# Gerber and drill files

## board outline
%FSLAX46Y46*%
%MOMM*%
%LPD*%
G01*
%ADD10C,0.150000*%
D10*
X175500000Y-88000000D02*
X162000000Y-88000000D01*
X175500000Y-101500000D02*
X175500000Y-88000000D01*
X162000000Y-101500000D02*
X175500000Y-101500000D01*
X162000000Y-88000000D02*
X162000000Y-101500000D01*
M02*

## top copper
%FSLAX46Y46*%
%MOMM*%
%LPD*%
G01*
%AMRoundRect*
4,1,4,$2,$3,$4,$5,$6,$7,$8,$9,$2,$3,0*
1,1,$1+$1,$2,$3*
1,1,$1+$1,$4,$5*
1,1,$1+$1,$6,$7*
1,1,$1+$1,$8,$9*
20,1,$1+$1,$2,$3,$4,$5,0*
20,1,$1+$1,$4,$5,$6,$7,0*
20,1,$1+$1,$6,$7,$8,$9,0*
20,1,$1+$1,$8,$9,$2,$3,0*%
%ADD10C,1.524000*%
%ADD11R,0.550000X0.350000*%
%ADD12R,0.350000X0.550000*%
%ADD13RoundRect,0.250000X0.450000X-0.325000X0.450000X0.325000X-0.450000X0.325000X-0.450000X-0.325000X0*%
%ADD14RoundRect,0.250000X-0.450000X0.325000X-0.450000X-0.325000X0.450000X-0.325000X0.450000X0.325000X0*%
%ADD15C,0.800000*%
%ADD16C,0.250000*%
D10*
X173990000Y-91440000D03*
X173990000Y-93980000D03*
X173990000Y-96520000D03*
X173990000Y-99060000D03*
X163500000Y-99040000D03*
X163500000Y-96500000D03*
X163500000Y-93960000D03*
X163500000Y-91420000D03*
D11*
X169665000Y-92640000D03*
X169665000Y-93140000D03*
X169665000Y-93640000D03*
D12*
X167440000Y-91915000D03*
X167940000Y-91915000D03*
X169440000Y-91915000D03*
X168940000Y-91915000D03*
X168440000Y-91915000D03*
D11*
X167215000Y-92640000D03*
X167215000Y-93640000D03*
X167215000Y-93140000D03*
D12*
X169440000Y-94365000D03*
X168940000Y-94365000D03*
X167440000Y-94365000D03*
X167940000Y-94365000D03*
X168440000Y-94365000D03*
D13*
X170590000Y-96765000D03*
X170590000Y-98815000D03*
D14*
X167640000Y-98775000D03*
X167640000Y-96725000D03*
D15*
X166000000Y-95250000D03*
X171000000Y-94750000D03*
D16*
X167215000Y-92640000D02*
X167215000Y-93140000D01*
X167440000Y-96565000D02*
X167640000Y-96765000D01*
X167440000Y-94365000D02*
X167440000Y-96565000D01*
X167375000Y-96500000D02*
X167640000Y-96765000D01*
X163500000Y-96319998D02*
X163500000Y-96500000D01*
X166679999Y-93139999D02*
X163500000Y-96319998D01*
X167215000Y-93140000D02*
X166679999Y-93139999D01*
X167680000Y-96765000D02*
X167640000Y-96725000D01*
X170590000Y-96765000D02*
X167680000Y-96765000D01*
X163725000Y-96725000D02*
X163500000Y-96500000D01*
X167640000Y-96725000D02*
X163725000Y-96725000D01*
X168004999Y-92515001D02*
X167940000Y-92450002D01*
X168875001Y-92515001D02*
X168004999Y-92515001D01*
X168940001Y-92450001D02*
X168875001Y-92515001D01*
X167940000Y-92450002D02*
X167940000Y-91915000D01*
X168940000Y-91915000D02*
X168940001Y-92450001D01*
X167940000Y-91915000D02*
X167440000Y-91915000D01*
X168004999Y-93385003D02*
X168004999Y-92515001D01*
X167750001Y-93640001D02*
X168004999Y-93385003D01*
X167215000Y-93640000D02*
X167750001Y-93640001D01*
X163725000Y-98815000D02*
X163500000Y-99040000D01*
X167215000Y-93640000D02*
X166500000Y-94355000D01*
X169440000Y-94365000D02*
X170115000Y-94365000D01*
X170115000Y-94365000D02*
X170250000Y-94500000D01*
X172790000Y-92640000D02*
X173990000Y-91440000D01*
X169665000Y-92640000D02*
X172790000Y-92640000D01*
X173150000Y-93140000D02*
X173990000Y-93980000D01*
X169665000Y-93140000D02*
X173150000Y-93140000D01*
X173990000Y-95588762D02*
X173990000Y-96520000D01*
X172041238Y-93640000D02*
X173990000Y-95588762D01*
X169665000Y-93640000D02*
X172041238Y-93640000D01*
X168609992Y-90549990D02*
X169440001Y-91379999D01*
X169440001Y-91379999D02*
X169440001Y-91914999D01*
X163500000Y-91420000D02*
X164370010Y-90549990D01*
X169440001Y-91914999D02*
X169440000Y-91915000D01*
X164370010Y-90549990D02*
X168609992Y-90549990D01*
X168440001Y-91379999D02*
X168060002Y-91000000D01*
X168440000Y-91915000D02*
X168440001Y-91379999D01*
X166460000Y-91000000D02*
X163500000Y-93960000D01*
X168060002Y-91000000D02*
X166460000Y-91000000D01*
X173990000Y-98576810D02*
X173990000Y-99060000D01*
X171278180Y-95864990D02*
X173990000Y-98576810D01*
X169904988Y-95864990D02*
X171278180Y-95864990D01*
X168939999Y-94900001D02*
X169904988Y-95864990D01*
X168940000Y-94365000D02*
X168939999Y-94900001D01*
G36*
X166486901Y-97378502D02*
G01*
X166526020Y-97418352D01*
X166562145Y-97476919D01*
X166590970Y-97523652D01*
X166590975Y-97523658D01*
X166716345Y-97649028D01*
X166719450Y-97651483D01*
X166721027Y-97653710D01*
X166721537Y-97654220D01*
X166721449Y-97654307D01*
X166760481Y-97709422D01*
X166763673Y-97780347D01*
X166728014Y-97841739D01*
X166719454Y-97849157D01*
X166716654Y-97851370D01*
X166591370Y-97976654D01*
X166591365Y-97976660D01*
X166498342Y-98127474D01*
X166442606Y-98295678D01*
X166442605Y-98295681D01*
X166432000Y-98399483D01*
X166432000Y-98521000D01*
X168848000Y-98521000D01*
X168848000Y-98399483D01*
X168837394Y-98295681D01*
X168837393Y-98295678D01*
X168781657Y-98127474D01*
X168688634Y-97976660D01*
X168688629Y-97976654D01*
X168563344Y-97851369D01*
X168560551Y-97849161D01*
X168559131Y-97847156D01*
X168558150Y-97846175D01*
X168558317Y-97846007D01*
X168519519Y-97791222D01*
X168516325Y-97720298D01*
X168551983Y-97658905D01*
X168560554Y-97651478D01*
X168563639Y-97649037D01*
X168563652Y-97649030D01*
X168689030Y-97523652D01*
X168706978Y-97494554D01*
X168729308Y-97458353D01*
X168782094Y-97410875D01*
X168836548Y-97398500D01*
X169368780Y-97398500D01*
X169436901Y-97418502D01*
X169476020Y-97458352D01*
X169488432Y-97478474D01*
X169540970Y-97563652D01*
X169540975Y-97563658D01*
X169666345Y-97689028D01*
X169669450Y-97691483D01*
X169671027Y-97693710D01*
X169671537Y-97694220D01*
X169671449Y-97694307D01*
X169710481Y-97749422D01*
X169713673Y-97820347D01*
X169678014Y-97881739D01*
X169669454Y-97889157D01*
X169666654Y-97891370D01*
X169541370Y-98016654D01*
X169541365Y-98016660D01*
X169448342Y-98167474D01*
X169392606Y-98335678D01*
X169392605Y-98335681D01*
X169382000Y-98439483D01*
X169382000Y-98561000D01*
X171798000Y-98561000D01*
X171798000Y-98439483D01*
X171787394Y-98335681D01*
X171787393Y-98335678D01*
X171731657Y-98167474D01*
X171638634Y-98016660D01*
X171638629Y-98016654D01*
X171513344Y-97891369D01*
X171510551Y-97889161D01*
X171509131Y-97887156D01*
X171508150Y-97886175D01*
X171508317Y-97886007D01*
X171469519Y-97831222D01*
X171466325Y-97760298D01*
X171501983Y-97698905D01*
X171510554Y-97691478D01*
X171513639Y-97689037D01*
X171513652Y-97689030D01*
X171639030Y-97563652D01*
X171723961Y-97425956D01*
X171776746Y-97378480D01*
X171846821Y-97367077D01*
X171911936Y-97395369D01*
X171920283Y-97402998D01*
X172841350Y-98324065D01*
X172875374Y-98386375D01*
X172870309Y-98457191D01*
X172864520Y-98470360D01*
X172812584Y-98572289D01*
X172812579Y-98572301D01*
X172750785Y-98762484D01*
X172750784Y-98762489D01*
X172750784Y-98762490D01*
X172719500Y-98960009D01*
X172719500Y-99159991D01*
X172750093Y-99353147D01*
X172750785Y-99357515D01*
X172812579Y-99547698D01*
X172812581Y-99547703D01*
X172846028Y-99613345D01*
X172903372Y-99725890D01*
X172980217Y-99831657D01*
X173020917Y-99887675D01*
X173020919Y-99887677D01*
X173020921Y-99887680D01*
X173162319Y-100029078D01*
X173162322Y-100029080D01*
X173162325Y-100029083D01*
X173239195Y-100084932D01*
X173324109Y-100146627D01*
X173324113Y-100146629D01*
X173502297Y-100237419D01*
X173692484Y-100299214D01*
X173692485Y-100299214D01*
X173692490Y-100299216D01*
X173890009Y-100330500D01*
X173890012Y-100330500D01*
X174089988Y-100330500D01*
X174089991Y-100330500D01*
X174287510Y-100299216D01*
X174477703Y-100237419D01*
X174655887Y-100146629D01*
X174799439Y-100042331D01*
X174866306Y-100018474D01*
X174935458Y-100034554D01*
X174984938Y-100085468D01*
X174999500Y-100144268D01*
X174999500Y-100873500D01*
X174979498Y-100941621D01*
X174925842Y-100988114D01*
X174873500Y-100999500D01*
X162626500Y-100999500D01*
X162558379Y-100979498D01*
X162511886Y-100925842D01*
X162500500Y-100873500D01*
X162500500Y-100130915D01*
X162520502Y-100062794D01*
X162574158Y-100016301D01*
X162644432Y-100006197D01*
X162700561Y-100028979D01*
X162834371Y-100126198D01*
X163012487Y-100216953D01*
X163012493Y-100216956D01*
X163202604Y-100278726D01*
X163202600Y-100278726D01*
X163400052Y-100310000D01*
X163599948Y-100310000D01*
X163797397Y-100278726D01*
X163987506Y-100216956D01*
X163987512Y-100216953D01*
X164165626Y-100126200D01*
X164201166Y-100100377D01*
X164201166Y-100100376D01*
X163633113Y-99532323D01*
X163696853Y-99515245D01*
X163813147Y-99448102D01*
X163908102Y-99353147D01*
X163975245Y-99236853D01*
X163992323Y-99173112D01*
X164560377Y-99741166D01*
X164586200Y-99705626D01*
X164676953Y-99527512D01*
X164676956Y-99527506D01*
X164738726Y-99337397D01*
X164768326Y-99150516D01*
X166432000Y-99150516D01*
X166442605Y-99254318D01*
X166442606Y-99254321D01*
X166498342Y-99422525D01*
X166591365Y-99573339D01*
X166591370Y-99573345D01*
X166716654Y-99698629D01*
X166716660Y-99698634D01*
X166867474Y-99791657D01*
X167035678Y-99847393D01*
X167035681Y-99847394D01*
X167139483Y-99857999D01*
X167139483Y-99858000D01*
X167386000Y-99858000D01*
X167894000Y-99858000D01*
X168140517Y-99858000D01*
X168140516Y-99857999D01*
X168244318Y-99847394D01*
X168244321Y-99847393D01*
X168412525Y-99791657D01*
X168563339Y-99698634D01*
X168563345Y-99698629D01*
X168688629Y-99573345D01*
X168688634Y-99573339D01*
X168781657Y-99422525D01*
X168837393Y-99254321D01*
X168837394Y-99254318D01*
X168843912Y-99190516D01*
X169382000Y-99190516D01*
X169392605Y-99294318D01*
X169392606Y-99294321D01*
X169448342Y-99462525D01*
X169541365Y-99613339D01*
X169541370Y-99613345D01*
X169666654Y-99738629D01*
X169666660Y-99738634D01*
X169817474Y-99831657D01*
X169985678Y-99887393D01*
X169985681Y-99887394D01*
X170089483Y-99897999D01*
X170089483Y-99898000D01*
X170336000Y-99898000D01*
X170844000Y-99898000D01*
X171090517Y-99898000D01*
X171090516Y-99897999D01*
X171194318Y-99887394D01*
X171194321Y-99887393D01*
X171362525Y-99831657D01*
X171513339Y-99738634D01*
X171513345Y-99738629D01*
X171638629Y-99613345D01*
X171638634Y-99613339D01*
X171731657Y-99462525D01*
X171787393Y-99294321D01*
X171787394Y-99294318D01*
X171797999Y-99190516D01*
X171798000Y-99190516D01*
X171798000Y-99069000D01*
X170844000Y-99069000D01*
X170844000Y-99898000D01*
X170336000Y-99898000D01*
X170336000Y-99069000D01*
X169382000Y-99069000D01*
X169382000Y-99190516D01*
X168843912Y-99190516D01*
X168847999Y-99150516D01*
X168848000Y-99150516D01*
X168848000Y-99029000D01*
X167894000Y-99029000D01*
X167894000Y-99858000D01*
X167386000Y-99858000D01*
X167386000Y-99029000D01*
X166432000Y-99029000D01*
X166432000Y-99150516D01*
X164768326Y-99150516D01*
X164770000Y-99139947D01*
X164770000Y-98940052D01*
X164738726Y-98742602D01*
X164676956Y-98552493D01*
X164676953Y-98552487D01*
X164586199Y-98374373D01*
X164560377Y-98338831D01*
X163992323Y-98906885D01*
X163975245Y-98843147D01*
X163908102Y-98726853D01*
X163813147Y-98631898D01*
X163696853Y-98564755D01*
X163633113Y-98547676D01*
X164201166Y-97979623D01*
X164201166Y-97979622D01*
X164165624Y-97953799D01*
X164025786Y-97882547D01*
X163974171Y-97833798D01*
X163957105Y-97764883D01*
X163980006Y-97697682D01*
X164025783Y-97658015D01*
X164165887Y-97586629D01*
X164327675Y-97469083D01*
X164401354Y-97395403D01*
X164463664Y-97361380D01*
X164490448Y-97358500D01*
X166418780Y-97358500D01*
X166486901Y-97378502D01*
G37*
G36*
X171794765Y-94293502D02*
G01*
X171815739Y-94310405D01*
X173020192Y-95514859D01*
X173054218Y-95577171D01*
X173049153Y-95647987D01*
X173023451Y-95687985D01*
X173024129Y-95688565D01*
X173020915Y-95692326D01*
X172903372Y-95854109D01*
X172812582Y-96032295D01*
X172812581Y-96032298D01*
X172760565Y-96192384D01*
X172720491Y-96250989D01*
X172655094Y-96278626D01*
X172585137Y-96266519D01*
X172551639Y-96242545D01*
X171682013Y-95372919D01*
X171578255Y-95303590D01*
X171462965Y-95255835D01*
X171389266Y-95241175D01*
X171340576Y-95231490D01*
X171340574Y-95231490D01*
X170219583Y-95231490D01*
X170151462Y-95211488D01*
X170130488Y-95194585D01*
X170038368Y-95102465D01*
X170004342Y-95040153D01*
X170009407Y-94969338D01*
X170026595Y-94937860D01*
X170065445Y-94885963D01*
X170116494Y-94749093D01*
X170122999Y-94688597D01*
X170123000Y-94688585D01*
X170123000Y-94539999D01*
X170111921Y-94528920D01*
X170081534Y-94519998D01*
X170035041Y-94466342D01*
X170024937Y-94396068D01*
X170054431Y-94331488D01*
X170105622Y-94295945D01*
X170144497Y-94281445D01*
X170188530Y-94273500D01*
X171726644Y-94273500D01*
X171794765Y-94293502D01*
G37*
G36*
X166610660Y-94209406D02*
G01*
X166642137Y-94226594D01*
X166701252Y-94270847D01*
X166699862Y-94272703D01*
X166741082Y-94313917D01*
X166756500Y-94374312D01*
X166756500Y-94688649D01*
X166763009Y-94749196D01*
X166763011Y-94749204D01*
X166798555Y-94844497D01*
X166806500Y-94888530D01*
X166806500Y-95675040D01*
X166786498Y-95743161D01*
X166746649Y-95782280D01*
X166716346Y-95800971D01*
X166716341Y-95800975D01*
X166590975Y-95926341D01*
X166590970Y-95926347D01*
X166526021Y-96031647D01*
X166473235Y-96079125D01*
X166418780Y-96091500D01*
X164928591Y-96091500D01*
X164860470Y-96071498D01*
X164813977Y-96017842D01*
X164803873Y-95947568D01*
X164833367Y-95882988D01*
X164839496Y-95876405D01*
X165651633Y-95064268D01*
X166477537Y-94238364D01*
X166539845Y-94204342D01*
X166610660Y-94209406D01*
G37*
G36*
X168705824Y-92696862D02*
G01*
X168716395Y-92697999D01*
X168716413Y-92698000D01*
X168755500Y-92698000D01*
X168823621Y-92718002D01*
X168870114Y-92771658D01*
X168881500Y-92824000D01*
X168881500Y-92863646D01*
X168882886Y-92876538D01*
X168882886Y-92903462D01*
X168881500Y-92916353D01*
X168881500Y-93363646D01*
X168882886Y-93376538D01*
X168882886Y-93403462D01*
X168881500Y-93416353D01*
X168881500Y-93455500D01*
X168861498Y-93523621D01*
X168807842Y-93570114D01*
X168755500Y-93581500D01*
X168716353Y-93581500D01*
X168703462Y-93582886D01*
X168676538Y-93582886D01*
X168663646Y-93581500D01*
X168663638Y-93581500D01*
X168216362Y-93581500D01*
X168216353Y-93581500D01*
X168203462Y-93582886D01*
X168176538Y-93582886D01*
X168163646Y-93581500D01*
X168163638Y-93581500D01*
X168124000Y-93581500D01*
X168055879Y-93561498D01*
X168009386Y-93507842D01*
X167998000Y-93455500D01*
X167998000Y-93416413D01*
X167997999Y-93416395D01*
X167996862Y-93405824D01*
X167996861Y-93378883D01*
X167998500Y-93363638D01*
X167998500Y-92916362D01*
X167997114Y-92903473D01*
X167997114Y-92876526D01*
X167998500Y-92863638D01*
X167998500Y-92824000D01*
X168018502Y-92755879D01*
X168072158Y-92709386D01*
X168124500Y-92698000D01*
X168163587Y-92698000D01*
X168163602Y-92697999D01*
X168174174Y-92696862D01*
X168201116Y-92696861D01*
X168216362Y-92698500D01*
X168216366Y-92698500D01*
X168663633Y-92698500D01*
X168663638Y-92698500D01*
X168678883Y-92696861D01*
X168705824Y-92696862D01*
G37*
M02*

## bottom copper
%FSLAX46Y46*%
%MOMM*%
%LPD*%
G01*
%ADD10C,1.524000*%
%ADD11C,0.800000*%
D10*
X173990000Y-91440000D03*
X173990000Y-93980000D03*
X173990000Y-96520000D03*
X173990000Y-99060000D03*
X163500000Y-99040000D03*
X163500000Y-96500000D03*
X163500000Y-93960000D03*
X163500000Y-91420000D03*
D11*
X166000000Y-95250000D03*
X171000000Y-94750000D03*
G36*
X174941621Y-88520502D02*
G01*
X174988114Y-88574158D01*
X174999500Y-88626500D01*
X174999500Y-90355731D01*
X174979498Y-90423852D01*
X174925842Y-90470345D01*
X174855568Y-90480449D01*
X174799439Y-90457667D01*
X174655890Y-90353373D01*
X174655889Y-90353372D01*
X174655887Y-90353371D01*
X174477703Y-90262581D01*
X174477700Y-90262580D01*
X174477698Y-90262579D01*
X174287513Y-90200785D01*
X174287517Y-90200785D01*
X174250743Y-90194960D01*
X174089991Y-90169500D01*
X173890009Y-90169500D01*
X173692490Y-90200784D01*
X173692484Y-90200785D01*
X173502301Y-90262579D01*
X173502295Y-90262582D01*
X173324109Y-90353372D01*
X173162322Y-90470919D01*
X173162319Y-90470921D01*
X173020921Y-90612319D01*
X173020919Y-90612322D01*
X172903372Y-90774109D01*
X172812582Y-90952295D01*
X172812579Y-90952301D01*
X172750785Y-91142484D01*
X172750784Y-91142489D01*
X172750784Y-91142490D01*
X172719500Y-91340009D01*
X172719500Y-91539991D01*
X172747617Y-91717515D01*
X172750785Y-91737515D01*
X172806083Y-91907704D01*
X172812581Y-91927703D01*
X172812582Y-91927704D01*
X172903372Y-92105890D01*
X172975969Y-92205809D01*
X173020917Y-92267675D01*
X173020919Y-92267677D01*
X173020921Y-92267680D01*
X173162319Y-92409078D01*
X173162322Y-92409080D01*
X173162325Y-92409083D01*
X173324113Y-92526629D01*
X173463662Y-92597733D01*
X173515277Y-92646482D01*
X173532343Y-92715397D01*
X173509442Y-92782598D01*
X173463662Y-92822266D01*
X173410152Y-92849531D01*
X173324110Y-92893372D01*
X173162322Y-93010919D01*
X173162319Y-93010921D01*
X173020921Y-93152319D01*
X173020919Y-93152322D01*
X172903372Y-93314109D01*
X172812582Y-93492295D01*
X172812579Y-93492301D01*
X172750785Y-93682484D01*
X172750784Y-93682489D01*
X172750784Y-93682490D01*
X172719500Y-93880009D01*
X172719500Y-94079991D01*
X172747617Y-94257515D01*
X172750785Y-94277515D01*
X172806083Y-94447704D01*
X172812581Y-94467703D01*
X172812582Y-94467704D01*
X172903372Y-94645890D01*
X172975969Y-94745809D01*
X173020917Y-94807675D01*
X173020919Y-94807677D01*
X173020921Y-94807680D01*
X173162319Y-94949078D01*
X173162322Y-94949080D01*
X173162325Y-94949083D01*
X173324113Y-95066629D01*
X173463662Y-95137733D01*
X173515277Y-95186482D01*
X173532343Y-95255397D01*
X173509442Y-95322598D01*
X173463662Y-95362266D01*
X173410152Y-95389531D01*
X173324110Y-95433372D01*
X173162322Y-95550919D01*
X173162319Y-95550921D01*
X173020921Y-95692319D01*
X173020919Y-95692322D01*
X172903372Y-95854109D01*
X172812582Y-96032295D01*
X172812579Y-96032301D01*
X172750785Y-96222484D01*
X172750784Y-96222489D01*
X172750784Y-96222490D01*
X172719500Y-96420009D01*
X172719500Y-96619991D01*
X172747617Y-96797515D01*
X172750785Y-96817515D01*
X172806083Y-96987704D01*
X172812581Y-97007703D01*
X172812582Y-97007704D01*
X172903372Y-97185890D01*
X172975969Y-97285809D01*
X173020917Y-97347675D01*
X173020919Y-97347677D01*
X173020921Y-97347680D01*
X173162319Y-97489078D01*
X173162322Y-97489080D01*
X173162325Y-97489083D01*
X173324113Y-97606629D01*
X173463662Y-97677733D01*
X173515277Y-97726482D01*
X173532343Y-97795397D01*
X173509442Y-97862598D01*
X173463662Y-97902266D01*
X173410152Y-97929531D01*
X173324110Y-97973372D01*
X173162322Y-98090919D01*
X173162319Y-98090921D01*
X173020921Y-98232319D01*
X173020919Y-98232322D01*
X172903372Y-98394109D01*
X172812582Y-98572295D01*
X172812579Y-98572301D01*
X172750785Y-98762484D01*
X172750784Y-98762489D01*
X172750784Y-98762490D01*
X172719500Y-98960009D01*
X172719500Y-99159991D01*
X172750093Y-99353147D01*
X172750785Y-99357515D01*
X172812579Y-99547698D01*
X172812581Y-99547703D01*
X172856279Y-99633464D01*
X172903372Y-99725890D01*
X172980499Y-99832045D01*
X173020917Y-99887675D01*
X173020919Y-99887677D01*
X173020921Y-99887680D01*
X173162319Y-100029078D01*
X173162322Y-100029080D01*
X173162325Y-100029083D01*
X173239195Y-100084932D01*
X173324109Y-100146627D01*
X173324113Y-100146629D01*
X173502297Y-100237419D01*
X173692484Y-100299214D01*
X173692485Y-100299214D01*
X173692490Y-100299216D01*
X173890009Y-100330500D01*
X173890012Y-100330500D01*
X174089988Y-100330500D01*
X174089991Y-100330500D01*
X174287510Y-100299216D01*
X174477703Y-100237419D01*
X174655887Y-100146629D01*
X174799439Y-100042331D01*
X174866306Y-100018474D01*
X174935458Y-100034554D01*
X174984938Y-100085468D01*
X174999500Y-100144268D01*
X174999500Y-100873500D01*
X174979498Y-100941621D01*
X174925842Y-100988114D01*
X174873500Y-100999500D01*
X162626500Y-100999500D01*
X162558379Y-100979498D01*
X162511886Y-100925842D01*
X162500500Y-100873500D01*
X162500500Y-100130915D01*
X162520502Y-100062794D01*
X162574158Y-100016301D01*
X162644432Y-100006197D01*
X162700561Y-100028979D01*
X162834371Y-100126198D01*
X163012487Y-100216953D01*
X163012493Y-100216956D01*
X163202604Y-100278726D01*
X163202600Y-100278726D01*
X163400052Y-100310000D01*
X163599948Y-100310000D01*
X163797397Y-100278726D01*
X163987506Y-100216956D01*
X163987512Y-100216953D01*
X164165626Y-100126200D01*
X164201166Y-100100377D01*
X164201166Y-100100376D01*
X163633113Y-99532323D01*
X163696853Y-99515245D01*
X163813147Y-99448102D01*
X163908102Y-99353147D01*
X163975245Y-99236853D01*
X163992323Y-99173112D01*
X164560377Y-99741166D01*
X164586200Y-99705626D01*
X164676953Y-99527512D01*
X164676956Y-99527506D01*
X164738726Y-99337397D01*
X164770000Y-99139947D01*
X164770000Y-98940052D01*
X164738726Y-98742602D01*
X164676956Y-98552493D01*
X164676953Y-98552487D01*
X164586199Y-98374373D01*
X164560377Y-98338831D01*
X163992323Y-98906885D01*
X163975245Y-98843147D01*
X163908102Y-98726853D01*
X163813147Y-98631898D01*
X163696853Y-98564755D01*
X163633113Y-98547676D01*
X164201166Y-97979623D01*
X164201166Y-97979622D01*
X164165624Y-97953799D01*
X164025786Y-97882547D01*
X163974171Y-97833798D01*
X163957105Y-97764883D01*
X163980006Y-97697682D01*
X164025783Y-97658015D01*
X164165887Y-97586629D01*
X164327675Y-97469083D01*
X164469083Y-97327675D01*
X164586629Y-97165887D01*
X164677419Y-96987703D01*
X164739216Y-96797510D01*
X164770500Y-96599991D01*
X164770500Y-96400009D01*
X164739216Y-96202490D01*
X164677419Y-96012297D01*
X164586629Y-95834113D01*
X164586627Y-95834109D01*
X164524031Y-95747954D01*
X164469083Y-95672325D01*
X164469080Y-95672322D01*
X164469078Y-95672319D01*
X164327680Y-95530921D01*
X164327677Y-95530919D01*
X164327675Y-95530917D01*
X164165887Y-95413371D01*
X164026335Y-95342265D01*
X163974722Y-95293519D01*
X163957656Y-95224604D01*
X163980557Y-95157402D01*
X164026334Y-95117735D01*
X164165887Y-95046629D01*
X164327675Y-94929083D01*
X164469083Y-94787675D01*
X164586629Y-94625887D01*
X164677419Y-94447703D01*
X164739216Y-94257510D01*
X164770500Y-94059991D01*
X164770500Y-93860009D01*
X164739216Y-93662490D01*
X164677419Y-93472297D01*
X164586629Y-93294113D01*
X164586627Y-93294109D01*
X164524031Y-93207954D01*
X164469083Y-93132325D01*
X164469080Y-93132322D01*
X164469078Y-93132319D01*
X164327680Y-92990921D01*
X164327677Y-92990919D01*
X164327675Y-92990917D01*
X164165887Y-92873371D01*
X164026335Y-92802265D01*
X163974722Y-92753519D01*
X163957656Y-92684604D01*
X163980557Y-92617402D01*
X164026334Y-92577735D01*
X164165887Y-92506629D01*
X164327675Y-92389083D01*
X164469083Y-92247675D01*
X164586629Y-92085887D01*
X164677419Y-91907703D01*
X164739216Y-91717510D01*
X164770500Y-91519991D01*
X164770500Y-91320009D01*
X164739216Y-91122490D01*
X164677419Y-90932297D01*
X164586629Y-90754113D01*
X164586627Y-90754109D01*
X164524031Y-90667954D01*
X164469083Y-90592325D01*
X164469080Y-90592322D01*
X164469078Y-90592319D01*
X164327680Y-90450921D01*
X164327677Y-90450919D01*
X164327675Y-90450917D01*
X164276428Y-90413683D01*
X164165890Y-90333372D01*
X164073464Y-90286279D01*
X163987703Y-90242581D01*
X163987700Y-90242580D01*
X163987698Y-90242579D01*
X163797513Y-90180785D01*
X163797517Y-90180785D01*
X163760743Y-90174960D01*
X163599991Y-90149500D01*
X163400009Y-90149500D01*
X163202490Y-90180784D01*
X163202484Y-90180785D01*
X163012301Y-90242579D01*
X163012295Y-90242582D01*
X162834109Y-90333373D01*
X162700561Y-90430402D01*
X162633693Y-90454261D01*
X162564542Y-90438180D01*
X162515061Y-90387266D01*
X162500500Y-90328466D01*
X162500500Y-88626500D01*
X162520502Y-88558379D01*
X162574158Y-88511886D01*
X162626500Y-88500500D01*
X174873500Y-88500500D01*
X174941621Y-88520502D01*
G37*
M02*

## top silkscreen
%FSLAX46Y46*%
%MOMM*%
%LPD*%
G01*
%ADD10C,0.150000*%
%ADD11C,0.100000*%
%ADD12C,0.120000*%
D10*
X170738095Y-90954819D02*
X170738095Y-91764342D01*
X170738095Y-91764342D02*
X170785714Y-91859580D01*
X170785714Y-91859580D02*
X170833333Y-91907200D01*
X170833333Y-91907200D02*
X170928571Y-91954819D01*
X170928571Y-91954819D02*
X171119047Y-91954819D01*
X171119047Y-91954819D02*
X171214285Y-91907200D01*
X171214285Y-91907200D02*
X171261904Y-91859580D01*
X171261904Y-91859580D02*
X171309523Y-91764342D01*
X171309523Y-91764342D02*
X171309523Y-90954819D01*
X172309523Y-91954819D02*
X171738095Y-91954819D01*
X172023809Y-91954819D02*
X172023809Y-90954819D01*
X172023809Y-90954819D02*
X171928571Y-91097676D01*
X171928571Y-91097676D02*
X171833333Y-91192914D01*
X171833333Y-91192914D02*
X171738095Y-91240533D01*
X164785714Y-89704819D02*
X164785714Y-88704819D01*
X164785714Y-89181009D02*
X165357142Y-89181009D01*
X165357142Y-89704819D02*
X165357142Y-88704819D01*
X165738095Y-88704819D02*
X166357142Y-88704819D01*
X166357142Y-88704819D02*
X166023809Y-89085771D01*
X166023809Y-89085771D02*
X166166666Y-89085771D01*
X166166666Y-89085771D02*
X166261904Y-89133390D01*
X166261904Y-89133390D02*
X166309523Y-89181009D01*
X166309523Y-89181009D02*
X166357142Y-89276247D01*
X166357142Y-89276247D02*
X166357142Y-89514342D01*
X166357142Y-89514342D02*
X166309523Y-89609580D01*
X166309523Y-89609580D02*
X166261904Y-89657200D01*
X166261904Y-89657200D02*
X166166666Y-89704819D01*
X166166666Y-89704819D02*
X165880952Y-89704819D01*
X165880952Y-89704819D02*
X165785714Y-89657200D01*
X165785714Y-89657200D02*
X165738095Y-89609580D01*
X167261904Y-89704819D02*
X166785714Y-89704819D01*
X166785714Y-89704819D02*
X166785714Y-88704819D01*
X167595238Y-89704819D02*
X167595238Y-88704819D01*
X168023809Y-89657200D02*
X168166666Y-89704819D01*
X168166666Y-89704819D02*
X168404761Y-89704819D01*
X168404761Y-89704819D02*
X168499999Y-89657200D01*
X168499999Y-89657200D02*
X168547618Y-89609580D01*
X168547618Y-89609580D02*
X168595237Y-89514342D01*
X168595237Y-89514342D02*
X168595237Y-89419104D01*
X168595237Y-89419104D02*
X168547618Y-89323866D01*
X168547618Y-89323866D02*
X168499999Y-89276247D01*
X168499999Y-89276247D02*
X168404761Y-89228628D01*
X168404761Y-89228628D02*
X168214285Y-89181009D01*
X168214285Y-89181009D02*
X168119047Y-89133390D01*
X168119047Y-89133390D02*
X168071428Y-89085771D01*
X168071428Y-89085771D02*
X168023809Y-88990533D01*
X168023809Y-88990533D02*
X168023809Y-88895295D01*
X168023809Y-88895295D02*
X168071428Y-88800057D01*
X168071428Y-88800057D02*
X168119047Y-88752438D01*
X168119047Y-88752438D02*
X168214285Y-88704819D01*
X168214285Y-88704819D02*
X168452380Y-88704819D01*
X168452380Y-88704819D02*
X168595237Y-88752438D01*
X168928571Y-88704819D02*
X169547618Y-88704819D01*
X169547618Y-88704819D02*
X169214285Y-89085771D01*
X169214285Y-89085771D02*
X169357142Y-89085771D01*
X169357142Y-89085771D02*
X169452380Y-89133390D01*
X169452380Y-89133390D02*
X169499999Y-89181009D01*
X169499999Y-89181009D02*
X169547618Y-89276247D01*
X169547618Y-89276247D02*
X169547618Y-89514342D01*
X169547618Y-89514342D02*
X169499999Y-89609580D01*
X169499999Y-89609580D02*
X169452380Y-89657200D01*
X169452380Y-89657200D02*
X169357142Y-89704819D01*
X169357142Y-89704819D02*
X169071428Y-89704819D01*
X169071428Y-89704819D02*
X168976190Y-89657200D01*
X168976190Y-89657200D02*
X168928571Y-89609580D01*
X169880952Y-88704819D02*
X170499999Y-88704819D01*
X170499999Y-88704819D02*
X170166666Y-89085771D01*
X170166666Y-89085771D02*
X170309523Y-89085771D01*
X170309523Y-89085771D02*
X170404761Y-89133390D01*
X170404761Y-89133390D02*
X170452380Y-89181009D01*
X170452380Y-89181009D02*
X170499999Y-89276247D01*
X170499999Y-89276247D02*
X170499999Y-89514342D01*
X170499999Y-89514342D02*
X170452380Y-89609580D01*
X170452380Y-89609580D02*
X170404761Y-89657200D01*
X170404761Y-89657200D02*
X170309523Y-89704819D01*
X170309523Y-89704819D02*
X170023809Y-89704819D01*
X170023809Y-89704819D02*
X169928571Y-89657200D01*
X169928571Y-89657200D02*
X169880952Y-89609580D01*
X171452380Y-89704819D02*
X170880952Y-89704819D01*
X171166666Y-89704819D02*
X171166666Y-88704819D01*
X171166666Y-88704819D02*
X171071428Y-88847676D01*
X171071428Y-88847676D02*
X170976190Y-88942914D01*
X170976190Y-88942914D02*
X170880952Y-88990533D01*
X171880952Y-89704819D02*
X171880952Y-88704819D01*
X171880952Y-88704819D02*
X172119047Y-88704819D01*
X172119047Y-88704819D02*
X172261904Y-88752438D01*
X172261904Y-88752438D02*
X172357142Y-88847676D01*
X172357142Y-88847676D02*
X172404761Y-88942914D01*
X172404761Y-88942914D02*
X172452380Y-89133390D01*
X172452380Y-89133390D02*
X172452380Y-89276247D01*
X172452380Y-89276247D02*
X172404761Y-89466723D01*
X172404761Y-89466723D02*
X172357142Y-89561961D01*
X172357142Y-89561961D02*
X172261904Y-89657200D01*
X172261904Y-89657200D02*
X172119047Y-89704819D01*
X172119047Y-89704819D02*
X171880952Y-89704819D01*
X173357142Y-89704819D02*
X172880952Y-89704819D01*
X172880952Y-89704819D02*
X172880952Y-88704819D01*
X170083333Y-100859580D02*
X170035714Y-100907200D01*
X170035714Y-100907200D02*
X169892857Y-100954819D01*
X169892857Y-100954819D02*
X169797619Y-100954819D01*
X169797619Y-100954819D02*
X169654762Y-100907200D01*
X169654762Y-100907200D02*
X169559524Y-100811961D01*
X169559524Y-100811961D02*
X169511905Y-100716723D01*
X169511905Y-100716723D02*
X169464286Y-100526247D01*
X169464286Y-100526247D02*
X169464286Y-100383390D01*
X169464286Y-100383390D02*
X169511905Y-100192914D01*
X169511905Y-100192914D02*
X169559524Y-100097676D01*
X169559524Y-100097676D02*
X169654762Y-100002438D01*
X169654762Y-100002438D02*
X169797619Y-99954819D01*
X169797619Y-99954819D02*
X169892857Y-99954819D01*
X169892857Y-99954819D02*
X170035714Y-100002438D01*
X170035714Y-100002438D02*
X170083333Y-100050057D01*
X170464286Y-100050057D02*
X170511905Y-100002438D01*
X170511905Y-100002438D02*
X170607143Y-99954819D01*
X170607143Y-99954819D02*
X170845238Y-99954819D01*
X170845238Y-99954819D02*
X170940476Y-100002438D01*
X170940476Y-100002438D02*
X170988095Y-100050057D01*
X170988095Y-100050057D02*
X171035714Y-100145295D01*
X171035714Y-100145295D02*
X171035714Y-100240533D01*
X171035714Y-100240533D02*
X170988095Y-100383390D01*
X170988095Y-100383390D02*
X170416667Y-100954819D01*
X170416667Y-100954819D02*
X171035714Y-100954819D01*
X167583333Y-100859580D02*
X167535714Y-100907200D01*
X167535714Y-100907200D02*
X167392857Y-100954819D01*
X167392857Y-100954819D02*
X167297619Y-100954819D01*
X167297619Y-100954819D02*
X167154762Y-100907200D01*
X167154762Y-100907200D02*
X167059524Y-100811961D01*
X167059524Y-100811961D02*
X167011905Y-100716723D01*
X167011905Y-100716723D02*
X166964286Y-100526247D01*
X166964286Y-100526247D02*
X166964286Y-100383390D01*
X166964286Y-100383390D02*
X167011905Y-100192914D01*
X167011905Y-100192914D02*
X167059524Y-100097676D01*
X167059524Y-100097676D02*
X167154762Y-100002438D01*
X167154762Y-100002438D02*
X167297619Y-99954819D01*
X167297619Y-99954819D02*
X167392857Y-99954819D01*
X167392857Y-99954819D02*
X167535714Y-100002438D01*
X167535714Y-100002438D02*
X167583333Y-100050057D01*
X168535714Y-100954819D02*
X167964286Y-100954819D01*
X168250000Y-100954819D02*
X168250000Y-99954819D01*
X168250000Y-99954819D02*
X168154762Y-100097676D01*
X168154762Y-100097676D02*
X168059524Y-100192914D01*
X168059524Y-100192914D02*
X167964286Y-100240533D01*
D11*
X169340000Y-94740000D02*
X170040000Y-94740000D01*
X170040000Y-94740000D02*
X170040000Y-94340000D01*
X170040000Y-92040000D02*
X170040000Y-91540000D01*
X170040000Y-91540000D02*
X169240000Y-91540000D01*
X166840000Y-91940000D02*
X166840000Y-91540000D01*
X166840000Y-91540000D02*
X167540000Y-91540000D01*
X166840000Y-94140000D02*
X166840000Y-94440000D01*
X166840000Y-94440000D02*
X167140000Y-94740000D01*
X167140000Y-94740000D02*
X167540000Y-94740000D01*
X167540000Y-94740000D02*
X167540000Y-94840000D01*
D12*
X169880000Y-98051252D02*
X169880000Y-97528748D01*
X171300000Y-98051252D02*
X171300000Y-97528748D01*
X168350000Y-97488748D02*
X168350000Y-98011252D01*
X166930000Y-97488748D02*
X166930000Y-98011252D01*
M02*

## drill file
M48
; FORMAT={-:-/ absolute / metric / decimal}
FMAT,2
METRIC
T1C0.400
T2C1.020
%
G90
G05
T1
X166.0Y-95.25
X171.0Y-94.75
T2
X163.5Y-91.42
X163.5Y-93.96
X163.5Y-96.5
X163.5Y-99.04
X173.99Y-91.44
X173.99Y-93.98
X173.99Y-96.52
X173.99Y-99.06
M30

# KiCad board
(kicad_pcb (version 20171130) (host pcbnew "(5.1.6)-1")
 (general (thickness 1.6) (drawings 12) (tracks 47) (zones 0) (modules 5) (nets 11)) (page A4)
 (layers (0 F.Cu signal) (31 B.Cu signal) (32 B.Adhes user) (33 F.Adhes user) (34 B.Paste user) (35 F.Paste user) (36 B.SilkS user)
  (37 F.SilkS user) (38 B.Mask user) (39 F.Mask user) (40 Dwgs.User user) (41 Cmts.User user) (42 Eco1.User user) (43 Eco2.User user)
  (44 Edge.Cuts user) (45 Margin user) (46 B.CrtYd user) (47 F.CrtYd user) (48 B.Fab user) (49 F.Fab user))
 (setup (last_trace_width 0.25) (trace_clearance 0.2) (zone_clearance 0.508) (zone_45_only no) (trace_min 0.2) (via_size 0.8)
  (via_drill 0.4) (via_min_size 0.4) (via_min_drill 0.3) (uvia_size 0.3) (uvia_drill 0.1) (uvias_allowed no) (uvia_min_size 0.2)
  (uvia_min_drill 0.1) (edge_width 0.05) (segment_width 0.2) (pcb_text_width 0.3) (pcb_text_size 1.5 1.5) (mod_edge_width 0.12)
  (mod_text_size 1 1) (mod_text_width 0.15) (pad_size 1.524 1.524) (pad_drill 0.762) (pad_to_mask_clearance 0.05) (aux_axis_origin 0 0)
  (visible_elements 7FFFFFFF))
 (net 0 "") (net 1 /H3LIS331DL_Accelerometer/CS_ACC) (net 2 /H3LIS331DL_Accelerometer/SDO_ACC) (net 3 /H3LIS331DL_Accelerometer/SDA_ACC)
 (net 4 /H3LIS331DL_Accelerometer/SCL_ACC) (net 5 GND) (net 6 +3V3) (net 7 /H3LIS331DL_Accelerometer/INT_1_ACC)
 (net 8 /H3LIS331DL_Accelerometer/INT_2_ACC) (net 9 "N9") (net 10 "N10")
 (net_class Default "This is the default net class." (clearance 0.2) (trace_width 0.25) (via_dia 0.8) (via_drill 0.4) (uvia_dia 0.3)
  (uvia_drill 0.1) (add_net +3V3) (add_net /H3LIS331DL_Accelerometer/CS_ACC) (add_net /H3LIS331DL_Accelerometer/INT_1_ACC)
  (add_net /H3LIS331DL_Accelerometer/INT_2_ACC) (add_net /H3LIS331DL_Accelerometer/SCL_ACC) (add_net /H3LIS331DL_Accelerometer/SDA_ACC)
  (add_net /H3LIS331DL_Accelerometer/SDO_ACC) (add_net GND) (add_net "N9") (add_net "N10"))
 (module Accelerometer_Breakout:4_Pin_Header (layer F.Cu) (at 173.99 99.06 180)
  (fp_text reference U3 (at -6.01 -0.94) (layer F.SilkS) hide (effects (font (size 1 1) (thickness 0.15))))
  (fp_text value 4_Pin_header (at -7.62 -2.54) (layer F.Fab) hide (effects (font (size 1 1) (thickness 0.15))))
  (pad 4 thru_hole circle (at 0 7.62 180) (size 1.524 1.524) (drill 1.02) (layers *.Cu *.Mask) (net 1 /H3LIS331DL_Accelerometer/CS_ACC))
  (pad 3 thru_hole circle (at 0 5.08 180) (size 1.524 1.524) (drill 1.02) (layers *.Cu *.Mask) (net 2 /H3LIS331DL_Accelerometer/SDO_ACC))
  (pad 2 thru_hole circle (at 0 2.54 180) (size 1.524 1.524) (drill 1.02) (layers *.Cu *.Mask) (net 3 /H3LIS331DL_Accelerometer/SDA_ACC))
  (pad 1 thru_hole circle (at 0 0 180) (size 1.524 1.524) (drill 1.02) (layers *.Cu *.Mask) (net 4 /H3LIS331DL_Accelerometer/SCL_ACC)))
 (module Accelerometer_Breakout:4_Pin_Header (layer F.Cu) (at 163.5 91.42)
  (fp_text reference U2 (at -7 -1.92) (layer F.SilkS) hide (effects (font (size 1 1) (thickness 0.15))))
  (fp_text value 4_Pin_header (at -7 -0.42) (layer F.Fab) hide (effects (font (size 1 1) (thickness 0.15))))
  (pad 4 thru_hole circle (at 0 7.62) (size 1.524 1.524) (drill 1.02) (layers *.Cu *.Mask) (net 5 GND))
  (pad 3 thru_hole circle (at 0 5.08) (size 1.524 1.524) (drill 1.02) (layers *.Cu *.Mask) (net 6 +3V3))
  (pad 2 thru_hole circle (at 0 2.54) (size 1.524 1.524) (drill 1.02) (layers *.Cu *.Mask) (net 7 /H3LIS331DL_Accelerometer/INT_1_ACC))
  (pad 1 thru_hole circle (at 0 0) (size 1.524 1.524) (drill 1.02) (layers *.Cu *.Mask) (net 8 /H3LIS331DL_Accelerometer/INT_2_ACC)))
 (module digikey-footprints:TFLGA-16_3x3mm (layer F.Cu) (at 168.44 93.14 90)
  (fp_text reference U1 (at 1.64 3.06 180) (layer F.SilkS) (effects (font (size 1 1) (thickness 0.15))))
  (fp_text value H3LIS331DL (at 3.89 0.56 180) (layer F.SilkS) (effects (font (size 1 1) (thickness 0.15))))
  (fp_line (start -1.6 0.9) (end -1.6 1.6) (layer F.SilkS) (width 0.1))
  (fp_line (start -1.6 1.6) (end -1.2 1.6) (layer F.SilkS) (width 0.1))
  (fp_line (start 1.1 1.6) (end 1.6 1.6) (layer F.SilkS) (width 0.1))
  (fp_line (start 1.6 1.6) (end 1.6 0.8) (layer F.SilkS) (width 0.1))
  (fp_line (start 1.2 -1.6) (end 1.6 -1.6) (layer F.SilkS) (width 0.1))
  (fp_line (start 1.6 -1.6) (end 1.6 -0.9) (layer F.SilkS) (width 0.1))
  (fp_line (start -1 -1.6) (end -1.3 -1.6) (layer F.SilkS) (width 0.1))
  (fp_line (start -1.3 -1.6) (end -1.6 -1.3) (layer F.SilkS) (width 0.1))
  (fp_line (start -1.6 -1.3) (end -1.6 -0.9) (layer F.SilkS) (width 0.1))
  (fp_line (start -1.6 -0.9) (end -1.7 -0.9) (layer F.SilkS) (width 0.1))
  (pad 8 smd rect (at 0.5 1.225 90) (size 0.35 0.55) (layers F.Cu F.Paste F.Mask) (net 1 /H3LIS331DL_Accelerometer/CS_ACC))
  (pad 7 smd rect (at 0 1.225 90) (size 0.35 0.55) (layers F.Cu F.Paste F.Mask) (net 2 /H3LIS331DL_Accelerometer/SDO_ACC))
  (pad 6 smd rect (at -0.5 1.225 90) (size 0.35 0.55) (layers F.Cu F.Paste F.Mask) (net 3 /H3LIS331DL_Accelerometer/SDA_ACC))
  (pad 13 smd rect (at 1.225 -1 90) (size 0.55 0.35) (layers F.Cu F.Paste F.Mask) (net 5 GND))
  (pad 12 smd rect (at 1.225 -0.5 90) (size 0.55 0.35) (layers F.Cu F.Paste F.Mask) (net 5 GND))
  (pad 9 smd rect (at 1.225 1 90) (size 0.55 0.35) (layers F.Cu F.Paste F.Mask) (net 8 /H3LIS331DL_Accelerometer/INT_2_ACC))
  (pad 10 smd rect (at 1.225 0.5 90) (size 0.55 0.35) (layers F.Cu F.Paste F.Mask) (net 5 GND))
  (pad 11 smd rect (at 1.225 0 90) (size 0.55 0.35) (layers F.Cu F.Paste F.Mask) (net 7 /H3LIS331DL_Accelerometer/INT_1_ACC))
  (pad 14 smd rect (at 0.5 -1.225 90) (size 0.35 0.55) (layers F.Cu F.Paste F.Mask) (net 6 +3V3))
  (pad 16 smd rect (at -0.5 -1.225 90) (size 0.35 0.55) (layers F.Cu F.Paste F.Mask) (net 5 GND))
  (pad 15 smd rect (at 0 -1.225 90) (size 0.35 0.55) (layers F.Cu F.Paste F.Mask) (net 6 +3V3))
  (pad 5 smd rect (at -1.225 1 90) (size 0.55 0.35) (layers F.Cu F.Paste F.Mask) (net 5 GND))
  (pad 4 smd rect (at -1.225 0.5 90) (size 0.55 0.35) (layers F.Cu F.Paste F.Mask) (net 4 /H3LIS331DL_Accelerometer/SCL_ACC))
  (pad 1 smd rect (at -1.225 -1 90) (size 0.55 0.35) (layers F.Cu F.Paste F.Mask) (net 6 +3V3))
  (pad 2 smd rect (at -1.225 -0.5 90) (size 0.55 0.35) (layers F.Cu F.Paste F.Mask) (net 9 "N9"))
  (pad 3 smd rect (at -1.225 0 90) (size 0.55 0.35) (layers F.Cu F.Paste F.Mask) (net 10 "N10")))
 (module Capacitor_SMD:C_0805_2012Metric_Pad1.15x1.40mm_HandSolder (layer F.Cu) (at 170.59 97.79 90)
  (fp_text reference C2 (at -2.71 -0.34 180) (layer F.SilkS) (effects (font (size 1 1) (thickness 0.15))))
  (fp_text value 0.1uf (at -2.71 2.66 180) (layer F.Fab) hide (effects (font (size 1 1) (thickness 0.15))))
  (fp_line (start -0.261252 -0.71) (end 0.261252 -0.71) (layer F.SilkS) (width 0.12))
  (fp_line (start -0.261252 0.71) (end 0.261252 0.71) (layer F.SilkS) (width 0.12))
  (pad 2 smd roundrect (at 1.025 0 90) (size 1.15 1.4) (layers F.Cu F.Paste F.Mask) (roundrect_rratio 0.217391) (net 6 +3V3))
  (pad 1 smd roundrect (at -1.025 0 90) (size 1.15 1.4) (layers F.Cu F.Paste F.Mask) (roundrect_rratio 0.217391) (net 5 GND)))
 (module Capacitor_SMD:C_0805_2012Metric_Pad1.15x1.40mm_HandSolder (layer F.Cu) (at 167.64 97.75 270)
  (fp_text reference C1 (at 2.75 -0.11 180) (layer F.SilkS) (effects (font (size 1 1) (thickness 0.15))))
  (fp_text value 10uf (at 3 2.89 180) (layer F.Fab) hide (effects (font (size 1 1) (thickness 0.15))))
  (fp_line (start -0.261252 -0.71) (end 0.261252 -0.71) (layer F.SilkS) (width 0.12))
  (fp_line (start -0.261252 0.71) (end 0.261252 0.71) (layer F.SilkS) (width 0.12))
  (pad 2 smd roundrect (at 1.025 0 270) (size 1.15 1.4) (layers F.Cu F.Paste F.Mask) (roundrect_rratio 0.217391) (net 5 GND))
  (pad 1 smd roundrect (at -1.025 0 270) (size 1.15 1.4) (layers F.Cu F.Paste F.Mask) (roundrect_rratio 0.217391) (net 6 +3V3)))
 (gr_line (start 175.5 88) (end 162 88) (layer Edge.Cuts) (width 0.15))
 (gr_line (start 175.5 101.5) (end 175.5 88) (layer Edge.Cuts) (width 0.15))
 (gr_line (start 162 101.5) (end 175.5 101.5) (layer Edge.Cuts) (width 0.15))
 (gr_line (start 162 88) (end 162 101.5) (layer Edge.Cuts) (width 0.15))
 (segment (start 167.215 92.64) (end 167.215 93.14) (width 0.25) (layer F.Cu) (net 6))
 (segment (start 167.44 96.565) (end 167.64 96.765) (width 0.25) (layer F.Cu) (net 6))
 (segment (start 167.44 94.365) (end 167.44 96.565) (width 0.25) (layer F.Cu) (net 6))
 (segment (start 167.375 96.5) (end 167.64 96.765) (width 0.25) (layer F.Cu) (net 6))
 (segment (start 163.5 96.319998) (end 163.5 96.5) (width 0.25) (layer F.Cu) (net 6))
 (segment (start 166.679999 93.139999) (end 163.5 96.319998) (width 0.25) (layer F.Cu) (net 6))
 (segment (start 167.215 93.14) (end 166.679999 93.139999) (width 0.25) (layer F.Cu) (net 6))
 (segment (start 167.68 96.765) (end 167.64 96.725) (width 0.25) (layer F.Cu) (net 6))
 (segment (start 170.59 96.765) (end 167.68 96.765) (width 0.25) (layer F.Cu) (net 6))
 (segment (start 163.725 96.725) (end 163.5 96.5) (width 0.25) (layer F.Cu) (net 6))
 (segment (start 167.64 96.725) (end 163.725 96.725) (width 0.25) (layer F.Cu) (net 6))
 (via (at 166 95.25) (size 0.8) (drill 0.4) (layers F.Cu B.Cu) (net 5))
 (via (at 171 94.75) (size 0.8) (drill 0.4) (layers F.Cu B.Cu) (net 5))
 (segment (start 168.004999 92.515001) (end 167.94 92.450002) (width 0.25) (layer F.Cu) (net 5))
 (segment (start 168.875001 92.515001) (end 168.004999 92.515001) (width 0.25) (layer F.Cu) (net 5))
 (segment (start 168.940001 92.450001) (end 168.875001 92.515001) (width 0.25) (layer F.Cu) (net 5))
 (segment (start 167.94 92.450002) (end 167.94 91.915) (width 0.25) (layer F.Cu) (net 5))
 (segment (start 168.94 91.915) (end 168.940001 92.450001) (width 0.25) (layer F.Cu) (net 5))
 (segment (start 167.94 91.915) (end 167.44 91.915) (width 0.25) (layer F.Cu) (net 5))
 (segment (start 168.004999 93.385003) (end 168.004999 92.515001) (width 0.25) (layer F.Cu) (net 5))
 (segment (start 167.750001 93.640001) (end 168.004999 93.385003) (width 0.25) (layer F.Cu) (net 5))
 (segment (start 167.215 93.64) (end 167.750001 93.640001) (width 0.25) (layer F.Cu) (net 5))
 (segment (start 163.725 98.815) (end 163.5 99.04) (width 0.25) (layer F.Cu) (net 5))
 (segment (start 167.215 93.64) (end 166.5 94.355) (width 0.25) (layer F.Cu) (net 5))
 (segment (start 169.44 94.365) (end 170.115 94.365) (width 0.25) (layer F.Cu) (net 5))
 (segment (start 170.115 94.365) (end 170.25 94.5) (width 0.25) (layer F.Cu) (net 5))
 (segment (start 172.79 92.64) (end 173.99 91.44) (width 0.25) (layer F.Cu) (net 1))
 (segment (start 169.665 92.64) (end 172.79 92.64) (width 0.25) (layer F.Cu) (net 1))
 (segment (start 173.15 93.14) (end 173.99 93.98) (width 0.25) (layer F.Cu) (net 2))
 (segment (start 169.665 93.14) (end 173.15 93.14) (width 0.25) (layer F.Cu) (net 2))
 (segment (start 173.99 95.588762) (end 173.99 96.52) (width 0.25) (layer F.Cu) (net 3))
 (segment (start 172.041238 93.64) (end 173.99 95.588762) (width 0.25) (layer F.Cu) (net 3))
 (segment (start 169.665 93.64) (end 172.041238 93.64) (width 0.25) (layer F.Cu) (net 3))
 (segment (start 168.609992 90.54999) (end 169.440001 91.379999) (width 0.25) (layer F.Cu) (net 8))
 (segment (start 169.440001 91.379999) (end 169.440001 91.914999) (width 0.25) (layer F.Cu) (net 8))
 (segment (start 163.5 91.42) (end 164.37001 90.54999) (width 0.25) (layer F.Cu) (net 8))
 (segment (start 169.440001 91.914999) (end 169.44 91.915) (width 0.25) (layer F.Cu) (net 8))
 (segment (start 164.37001 90.54999) (end 168.609992 90.54999) (width 0.25) (layer F.Cu) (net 8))
 (segment (start 168.440001 91.379999) (end 168.060002 91) (width 0.25) (layer F.Cu) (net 7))
 (segment (start 168.44 91.915) (end 168.440001 91.379999) (width 0.25) (layer F.Cu) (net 7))
 (segment (start 166.46 91) (end 163.5 93.96) (width 0.25) (layer F.Cu) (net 7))
 (segment (start 168.060002 91) (end 166.46 91) (width 0.25) (layer F.Cu) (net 7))
 (segment (start 173.99 98.57681) (end 173.99 99.06) (width 0.25) (layer F.Cu) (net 4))
 (segment (start 171.27818 95.86499) (end 173.99 98.57681) (width 0.25) (layer F.Cu) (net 4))
 (segment (start 169.904988 95.86499) (end 171.27818 95.86499) (width 0.25) (layer F.Cu) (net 4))
 (segment (start 168.939999 94.900001) (end 169.904988 95.86499) (width 0.25) (layer F.Cu) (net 4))
 (segment (start 168.94 94.365) (end 168.939999 94.900001) (width 0.25) (layer F.Cu) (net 4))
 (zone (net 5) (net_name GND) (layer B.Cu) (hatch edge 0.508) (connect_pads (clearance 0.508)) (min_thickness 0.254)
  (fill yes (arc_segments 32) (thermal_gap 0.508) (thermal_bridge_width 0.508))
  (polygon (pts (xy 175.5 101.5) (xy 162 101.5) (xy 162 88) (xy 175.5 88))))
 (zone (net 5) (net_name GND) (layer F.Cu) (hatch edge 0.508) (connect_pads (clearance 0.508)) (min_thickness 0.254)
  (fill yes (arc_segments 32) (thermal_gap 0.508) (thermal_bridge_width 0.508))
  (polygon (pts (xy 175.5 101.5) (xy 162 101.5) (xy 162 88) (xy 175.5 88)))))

